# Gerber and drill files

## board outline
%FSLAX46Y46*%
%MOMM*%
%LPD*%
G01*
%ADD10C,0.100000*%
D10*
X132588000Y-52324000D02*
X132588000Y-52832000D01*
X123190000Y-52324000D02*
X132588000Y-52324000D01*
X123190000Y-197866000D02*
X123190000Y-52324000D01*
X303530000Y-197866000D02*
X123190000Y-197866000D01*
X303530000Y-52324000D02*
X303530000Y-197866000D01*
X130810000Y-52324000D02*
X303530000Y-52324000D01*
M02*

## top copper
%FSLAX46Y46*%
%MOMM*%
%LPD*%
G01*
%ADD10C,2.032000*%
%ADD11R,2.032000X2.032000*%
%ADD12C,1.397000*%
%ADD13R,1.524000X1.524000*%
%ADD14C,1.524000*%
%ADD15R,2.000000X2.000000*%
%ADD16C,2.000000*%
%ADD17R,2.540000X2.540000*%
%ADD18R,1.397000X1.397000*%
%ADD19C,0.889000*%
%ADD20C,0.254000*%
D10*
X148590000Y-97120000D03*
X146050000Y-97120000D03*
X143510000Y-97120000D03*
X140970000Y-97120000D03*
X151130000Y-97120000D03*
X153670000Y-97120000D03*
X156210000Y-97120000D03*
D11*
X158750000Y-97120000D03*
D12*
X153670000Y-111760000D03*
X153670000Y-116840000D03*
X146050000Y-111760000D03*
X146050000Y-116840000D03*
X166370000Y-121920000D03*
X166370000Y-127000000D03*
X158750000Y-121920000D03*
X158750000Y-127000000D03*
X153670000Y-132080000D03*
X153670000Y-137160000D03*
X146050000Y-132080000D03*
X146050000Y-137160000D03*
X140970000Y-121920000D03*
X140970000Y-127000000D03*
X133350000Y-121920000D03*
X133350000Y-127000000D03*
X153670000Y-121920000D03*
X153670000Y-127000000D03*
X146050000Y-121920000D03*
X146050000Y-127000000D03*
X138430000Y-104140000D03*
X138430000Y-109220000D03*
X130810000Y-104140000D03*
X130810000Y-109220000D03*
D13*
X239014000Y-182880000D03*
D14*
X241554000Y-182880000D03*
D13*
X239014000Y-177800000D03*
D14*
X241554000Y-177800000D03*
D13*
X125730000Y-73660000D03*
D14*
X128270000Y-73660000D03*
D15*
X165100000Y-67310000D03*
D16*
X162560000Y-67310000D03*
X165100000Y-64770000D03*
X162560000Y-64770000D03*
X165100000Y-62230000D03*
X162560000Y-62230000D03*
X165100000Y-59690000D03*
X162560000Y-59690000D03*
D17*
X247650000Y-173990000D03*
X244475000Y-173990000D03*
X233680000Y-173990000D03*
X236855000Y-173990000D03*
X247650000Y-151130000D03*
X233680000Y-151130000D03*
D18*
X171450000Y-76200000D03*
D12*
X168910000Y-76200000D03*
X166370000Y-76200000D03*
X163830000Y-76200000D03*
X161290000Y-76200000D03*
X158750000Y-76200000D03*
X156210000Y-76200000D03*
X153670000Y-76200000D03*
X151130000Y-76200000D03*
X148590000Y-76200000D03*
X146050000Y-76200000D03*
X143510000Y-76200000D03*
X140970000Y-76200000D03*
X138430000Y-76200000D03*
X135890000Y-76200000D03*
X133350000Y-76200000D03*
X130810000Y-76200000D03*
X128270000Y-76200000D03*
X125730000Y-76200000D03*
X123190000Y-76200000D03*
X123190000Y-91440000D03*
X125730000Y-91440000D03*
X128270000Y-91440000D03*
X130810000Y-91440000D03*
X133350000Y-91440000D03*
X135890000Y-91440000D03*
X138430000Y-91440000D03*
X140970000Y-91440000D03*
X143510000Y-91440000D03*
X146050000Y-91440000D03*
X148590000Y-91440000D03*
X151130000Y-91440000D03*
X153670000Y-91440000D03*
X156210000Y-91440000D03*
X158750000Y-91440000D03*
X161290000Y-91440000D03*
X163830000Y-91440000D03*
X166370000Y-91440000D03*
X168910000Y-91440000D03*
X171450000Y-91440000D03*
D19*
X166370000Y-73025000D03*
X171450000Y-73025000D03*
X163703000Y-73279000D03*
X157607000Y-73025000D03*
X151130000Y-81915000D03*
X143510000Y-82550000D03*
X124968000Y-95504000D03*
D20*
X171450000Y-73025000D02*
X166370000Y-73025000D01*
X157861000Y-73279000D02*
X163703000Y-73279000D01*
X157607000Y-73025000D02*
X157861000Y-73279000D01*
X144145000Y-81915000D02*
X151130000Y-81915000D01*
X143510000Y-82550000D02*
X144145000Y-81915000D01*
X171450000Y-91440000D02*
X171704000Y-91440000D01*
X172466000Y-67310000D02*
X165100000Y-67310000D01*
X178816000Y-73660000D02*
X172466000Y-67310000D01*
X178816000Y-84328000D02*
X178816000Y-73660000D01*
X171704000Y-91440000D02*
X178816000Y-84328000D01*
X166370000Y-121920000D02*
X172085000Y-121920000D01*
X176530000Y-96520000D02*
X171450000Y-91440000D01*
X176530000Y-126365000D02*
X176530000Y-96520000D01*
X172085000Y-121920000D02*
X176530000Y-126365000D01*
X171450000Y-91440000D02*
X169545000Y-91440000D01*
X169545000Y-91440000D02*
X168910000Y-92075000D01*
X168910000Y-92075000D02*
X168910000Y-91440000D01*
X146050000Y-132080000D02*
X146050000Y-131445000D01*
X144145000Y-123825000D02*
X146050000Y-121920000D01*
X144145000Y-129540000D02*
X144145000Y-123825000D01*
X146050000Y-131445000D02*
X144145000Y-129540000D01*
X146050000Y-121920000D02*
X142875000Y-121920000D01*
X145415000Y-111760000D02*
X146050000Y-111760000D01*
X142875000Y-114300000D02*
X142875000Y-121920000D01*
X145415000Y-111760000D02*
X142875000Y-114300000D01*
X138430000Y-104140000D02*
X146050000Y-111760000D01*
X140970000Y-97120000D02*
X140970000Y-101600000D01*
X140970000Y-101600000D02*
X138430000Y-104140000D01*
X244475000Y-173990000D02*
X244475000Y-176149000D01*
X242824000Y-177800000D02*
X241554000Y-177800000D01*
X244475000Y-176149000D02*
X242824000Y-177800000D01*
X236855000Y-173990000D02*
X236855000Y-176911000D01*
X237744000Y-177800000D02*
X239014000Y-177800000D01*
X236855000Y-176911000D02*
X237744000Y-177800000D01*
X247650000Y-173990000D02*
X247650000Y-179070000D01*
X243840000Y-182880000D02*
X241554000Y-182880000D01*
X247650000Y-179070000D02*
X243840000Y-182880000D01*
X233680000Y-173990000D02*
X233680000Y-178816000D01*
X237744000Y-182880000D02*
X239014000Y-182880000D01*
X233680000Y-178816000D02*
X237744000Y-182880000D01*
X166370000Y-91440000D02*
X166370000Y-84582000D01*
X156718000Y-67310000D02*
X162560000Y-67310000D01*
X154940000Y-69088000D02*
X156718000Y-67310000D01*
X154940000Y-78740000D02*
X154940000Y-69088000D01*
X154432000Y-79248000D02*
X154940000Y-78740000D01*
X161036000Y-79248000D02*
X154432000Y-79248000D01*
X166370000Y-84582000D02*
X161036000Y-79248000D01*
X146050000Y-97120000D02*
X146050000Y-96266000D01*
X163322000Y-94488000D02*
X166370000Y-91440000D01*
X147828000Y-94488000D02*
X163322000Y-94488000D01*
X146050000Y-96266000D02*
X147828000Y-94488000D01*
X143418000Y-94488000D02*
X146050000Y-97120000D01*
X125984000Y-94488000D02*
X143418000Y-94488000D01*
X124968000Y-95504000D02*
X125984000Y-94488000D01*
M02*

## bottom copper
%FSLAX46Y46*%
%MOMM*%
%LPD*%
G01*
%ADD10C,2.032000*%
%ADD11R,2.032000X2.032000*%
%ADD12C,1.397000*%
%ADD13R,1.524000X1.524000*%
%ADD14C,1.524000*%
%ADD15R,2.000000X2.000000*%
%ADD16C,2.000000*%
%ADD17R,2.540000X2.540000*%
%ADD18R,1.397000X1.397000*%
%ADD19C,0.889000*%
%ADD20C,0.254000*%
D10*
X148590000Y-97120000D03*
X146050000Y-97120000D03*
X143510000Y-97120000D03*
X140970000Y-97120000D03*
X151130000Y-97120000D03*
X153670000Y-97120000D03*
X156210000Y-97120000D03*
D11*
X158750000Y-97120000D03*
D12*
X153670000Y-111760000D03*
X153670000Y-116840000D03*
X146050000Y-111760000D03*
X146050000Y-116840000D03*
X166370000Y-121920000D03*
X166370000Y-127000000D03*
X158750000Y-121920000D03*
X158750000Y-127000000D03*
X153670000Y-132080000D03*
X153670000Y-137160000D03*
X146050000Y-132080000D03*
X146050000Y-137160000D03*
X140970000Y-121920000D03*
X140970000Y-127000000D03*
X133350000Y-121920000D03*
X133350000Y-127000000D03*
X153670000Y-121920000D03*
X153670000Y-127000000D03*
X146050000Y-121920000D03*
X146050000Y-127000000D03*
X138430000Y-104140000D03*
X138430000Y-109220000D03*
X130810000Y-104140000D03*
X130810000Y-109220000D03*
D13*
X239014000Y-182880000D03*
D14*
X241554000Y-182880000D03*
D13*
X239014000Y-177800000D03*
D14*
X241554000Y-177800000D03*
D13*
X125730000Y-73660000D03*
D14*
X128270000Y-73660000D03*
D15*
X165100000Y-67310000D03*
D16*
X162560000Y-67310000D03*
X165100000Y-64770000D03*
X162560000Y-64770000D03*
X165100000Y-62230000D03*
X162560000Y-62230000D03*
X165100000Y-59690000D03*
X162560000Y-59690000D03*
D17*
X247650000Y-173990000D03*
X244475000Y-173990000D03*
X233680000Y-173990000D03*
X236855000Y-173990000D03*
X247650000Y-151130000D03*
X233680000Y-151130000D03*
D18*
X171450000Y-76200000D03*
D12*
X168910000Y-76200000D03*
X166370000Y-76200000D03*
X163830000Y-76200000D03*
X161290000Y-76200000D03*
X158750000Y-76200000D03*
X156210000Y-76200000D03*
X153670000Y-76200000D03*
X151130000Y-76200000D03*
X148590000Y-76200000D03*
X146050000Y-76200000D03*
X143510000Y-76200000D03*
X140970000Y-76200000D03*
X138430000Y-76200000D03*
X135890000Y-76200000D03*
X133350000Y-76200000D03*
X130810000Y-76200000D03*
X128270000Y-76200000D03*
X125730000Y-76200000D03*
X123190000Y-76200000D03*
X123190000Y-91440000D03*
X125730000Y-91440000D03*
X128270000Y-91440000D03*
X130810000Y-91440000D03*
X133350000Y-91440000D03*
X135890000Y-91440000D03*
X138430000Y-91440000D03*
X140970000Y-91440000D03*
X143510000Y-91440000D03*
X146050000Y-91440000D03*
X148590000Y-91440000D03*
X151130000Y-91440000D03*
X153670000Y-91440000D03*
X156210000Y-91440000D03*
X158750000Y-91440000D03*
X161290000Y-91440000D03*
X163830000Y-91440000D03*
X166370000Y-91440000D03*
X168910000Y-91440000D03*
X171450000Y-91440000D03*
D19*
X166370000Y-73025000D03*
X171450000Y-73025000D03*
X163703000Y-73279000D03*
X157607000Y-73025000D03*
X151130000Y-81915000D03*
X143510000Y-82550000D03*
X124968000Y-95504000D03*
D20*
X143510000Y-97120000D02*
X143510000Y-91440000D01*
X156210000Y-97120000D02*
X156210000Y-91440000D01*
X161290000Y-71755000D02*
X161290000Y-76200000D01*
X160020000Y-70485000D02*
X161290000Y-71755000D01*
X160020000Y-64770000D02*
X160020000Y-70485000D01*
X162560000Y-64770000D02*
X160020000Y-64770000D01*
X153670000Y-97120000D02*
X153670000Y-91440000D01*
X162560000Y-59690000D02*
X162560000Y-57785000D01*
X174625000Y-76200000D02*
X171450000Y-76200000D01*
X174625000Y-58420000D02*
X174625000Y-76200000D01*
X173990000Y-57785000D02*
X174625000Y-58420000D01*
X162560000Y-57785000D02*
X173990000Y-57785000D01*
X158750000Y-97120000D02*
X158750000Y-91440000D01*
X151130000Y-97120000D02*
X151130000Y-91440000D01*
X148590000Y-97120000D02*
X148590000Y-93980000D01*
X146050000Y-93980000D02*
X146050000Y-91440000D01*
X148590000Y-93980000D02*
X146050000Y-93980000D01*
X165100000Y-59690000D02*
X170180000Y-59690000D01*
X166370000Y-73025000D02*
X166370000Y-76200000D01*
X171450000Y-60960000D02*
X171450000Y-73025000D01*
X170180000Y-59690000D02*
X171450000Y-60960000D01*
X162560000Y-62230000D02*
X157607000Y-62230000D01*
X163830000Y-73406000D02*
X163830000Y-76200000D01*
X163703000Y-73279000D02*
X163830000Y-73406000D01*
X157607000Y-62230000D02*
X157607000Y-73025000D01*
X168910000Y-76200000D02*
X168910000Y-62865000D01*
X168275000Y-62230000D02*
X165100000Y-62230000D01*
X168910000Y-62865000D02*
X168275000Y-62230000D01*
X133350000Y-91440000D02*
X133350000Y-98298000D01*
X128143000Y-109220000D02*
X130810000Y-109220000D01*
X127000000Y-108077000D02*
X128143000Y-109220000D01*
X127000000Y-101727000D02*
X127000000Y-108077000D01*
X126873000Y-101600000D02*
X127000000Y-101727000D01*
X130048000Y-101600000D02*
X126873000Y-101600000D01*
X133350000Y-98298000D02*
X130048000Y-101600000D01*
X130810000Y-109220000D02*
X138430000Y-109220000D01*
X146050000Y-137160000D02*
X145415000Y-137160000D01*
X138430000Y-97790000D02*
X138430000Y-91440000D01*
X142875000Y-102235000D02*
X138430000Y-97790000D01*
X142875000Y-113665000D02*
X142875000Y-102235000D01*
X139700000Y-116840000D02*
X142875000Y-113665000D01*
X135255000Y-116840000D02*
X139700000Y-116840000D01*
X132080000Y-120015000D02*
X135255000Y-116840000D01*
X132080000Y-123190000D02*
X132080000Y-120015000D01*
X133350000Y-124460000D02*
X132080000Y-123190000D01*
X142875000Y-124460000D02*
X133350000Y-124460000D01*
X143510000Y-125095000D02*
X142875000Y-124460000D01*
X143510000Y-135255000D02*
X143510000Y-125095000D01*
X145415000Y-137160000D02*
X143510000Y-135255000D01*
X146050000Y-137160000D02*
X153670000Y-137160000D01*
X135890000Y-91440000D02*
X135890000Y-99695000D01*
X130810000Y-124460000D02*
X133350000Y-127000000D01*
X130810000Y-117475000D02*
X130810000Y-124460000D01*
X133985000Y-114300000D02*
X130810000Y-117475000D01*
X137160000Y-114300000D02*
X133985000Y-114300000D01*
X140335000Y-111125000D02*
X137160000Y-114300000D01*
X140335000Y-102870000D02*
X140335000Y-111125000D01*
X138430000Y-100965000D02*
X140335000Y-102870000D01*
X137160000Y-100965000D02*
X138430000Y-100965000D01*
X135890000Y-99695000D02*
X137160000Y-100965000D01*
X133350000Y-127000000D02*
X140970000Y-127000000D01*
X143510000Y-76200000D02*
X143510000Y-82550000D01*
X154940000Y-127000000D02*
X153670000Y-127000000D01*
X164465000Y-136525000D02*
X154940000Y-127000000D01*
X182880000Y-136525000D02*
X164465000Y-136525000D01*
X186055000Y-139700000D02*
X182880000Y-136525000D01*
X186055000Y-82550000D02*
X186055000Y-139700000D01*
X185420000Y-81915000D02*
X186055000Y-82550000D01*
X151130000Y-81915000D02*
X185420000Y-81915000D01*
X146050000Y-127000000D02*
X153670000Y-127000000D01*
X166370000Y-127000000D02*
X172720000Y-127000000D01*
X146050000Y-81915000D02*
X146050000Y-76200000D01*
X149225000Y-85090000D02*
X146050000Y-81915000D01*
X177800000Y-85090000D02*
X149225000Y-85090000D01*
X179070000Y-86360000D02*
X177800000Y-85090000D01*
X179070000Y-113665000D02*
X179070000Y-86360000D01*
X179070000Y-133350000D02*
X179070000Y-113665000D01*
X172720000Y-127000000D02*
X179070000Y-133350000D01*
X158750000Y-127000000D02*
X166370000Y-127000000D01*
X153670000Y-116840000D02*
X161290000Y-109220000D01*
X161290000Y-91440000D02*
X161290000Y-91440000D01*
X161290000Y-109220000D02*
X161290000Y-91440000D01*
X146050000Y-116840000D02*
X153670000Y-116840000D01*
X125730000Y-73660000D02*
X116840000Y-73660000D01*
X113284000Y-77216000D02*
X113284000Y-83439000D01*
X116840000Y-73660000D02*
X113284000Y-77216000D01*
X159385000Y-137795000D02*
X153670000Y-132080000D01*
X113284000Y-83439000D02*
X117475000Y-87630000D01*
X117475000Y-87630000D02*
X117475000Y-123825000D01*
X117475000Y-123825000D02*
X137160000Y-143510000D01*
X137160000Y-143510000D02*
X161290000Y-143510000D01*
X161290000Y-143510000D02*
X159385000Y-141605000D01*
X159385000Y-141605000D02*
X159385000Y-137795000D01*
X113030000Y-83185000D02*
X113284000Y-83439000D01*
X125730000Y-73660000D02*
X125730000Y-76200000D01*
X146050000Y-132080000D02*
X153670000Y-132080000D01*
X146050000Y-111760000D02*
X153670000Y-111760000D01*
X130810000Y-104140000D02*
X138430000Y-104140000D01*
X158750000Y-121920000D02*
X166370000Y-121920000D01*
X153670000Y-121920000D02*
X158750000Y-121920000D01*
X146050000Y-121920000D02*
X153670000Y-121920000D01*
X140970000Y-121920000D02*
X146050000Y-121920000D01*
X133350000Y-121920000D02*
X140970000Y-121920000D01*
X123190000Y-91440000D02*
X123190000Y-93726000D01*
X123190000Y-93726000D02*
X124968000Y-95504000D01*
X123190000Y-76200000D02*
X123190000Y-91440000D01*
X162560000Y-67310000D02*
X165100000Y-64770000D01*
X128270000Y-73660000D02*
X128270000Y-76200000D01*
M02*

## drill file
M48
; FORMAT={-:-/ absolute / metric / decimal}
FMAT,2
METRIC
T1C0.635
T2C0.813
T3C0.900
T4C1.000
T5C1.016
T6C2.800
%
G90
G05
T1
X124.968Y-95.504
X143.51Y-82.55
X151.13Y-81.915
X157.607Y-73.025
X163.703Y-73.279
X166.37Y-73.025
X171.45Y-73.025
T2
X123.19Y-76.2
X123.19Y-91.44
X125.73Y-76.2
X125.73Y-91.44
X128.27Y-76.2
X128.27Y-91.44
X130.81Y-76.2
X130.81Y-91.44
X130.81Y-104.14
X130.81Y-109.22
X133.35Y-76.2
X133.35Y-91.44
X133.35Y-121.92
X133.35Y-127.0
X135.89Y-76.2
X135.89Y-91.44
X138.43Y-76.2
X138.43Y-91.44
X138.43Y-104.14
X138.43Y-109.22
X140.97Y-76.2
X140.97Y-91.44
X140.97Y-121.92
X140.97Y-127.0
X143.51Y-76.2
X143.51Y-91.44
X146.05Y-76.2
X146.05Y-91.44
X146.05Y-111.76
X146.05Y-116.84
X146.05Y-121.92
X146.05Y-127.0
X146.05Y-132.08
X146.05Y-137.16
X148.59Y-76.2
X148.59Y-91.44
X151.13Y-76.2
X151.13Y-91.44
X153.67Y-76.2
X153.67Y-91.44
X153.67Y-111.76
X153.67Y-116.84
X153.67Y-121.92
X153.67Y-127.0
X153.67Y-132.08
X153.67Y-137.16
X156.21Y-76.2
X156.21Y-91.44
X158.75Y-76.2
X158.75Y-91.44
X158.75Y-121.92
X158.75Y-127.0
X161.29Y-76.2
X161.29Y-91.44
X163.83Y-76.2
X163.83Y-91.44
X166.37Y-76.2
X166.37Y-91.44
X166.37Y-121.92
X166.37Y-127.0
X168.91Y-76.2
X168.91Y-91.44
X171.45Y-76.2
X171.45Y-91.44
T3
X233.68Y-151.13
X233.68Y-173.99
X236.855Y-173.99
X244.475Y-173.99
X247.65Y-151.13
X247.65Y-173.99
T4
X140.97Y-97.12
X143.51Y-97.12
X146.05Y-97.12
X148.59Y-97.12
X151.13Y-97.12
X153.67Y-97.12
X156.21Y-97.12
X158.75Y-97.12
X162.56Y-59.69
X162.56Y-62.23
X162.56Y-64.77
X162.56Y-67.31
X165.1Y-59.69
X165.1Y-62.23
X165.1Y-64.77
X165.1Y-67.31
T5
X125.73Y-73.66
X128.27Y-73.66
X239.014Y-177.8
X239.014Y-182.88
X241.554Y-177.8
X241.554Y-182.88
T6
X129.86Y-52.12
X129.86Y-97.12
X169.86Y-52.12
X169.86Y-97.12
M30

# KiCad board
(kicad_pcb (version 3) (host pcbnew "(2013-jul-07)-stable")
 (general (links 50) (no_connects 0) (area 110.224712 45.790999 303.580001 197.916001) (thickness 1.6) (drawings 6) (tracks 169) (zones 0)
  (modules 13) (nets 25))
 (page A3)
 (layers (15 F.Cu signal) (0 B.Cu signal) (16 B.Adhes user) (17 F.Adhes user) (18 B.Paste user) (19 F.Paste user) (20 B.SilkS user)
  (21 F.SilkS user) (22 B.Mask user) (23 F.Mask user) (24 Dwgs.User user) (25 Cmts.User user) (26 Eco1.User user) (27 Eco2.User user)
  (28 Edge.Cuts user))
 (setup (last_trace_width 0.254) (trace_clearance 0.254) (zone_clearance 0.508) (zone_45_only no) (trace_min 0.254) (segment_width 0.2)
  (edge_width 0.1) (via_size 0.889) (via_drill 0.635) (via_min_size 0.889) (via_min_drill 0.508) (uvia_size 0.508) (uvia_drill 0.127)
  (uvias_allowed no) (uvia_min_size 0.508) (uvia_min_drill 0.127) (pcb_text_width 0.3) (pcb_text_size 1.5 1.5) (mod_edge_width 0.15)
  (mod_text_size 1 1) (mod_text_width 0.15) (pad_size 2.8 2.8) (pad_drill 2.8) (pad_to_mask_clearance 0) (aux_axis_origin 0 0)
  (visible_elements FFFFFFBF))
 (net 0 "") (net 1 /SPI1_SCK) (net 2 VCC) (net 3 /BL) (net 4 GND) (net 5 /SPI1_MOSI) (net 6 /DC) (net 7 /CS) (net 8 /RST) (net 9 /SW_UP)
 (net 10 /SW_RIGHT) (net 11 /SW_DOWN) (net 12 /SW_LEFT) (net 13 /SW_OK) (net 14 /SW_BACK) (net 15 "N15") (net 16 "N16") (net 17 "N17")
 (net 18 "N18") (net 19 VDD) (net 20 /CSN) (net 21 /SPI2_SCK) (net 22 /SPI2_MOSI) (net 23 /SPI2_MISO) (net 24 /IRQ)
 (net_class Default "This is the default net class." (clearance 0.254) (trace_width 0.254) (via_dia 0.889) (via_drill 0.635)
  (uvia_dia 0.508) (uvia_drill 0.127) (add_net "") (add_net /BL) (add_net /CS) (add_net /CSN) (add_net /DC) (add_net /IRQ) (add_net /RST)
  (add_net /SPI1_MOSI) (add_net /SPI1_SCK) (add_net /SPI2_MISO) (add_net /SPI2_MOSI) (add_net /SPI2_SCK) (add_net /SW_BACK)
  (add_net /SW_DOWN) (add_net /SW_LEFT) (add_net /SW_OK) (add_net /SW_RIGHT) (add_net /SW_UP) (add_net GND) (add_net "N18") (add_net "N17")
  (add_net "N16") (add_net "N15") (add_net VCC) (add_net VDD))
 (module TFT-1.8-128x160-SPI (layer F.Cu) (at 149.86 71.12 270)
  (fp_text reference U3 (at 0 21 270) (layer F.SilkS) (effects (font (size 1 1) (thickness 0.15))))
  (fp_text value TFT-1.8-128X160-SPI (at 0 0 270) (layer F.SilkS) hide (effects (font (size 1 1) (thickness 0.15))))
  (pad 5 thru_hole circle (at 26 1.27 270) (size 2.032 2.032) (drill 1) (layers *.Cu *.Mask F.SilkS) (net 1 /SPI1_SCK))
  (pad 6 thru_hole circle (at 26 3.81 270) (size 2.032 2.032) (drill 1) (layers *.Cu *.Mask F.SilkS) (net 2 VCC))
  (pad 7 thru_hole circle (at 26 6.35 270) (size 2.032 2.032) (drill 1) (layers *.Cu *.Mask F.SilkS) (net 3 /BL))
  (pad 8 thru_hole circle (at 26 8.89 270) (size 2.032 2.032) (drill 1) (layers *.Cu *.Mask F.SilkS) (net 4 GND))
  (pad 4 thru_hole circle (at 26 -1.27 270) (size 2.032 2.032) (drill 1) (layers *.Cu *.Mask F.SilkS) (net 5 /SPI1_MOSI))
  (pad 3 thru_hole circle (at 26 -3.81 270) (size 2.032 2.032) (drill 1) (layers *.Cu *.Mask F.SilkS) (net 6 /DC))
  (pad 2 thru_hole circle (at 26 -6.35 270) (size 2.032 2.032) (drill 1) (layers *.Cu *.Mask F.SilkS) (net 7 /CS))
  (pad 1 thru_hole rect (at 26 -8.89 270) (size 2.032 2.032) (drill 1) (layers *.Cu *.Mask F.SilkS) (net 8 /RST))
  (pad "" np_thru_hole circle (at -19 20 270) (size 2.8 2.8) (drill 2.8) (layers *.Cu *.Mask F.SilkS))
  (pad "" np_thru_hole circle (at 26 20 270) (size 2.8 2.8) (drill 2.8) (layers *.Cu *.Mask F.SilkS))
  (pad "" np_thru_hole circle (at 26 -20 270) (size 2.8 2.8) (drill 2.8) (layers *.Cu *.Mask F.SilkS))
  (pad "" np_thru_hole circle (at -19 -20 270) (size 2.8 2.8) (drill 2.8) (layers *.Cu *.Mask F.SilkS)))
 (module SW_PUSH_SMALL (layer F.Cu) (at 149.86 114.3)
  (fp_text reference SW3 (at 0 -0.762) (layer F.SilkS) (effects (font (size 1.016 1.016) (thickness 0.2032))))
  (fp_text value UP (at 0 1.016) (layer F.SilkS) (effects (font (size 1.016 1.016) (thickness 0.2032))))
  (pad 1 thru_hole circle (at 3.81 -2.54) (size 1.397 1.397) (drill 0.8128) (layers *.Cu *.Mask F.SilkS) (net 4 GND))
  (pad 2 thru_hole circle (at 3.81 2.54) (size 1.397 1.397) (drill 0.8128) (layers *.Cu *.Mask F.SilkS) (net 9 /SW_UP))
  (pad 1 thru_hole circle (at -3.81 -2.54) (size 1.397 1.397) (drill 0.8128) (layers *.Cu *.Mask F.SilkS) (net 4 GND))
  (pad 2 thru_hole circle (at -3.81 2.54) (size 1.397 1.397) (drill 0.8128) (layers *.Cu *.Mask F.SilkS) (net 9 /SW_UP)))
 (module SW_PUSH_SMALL (layer F.Cu) (at 162.56 124.46)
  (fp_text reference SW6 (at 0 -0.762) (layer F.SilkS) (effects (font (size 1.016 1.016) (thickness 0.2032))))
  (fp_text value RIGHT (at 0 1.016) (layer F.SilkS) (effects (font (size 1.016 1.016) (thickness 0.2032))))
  (pad 1 thru_hole circle (at 3.81 -2.54) (size 1.397 1.397) (drill 0.8128) (layers *.Cu *.Mask F.SilkS) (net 4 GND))
  (pad 2 thru_hole circle (at 3.81 2.54) (size 1.397 1.397) (drill 0.8128) (layers *.Cu *.Mask F.SilkS) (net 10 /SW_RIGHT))
  (pad 1 thru_hole circle (at -3.81 -2.54) (size 1.397 1.397) (drill 0.8128) (layers *.Cu *.Mask F.SilkS) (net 4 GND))
  (pad 2 thru_hole circle (at -3.81 2.54) (size 1.397 1.397) (drill 0.8128) (layers *.Cu *.Mask F.SilkS) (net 10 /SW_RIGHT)))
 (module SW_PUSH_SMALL (layer F.Cu) (at 149.86 134.62)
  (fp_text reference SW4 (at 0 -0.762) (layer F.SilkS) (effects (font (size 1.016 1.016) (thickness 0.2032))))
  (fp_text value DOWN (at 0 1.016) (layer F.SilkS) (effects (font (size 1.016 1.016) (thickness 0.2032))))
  (pad 1 thru_hole circle (at 3.81 -2.54) (size 1.397 1.397) (drill 0.8128) (layers *.Cu *.Mask F.SilkS) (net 4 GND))
  (pad 2 thru_hole circle (at 3.81 2.54) (size 1.397 1.397) (drill 0.8128) (layers *.Cu *.Mask F.SilkS) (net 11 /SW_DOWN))
  (pad 1 thru_hole circle (at -3.81 -2.54) (size 1.397 1.397) (drill 0.8128) (layers *.Cu *.Mask F.SilkS) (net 4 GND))
  (pad 2 thru_hole circle (at -3.81 2.54) (size 1.397 1.397) (drill 0.8128) (layers *.Cu *.Mask F.SilkS) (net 11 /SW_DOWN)))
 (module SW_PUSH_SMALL (layer F.Cu) (at 137.16 124.46)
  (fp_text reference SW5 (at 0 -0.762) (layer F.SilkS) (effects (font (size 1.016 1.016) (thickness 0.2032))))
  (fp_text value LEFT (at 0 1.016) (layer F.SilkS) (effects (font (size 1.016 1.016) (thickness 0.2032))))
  (pad 1 thru_hole circle (at 3.81 -2.54) (size 1.397 1.397) (drill 0.8128) (layers *.Cu *.Mask F.SilkS) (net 4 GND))
  (pad 2 thru_hole circle (at 3.81 2.54) (size 1.397 1.397) (drill 0.8128) (layers *.Cu *.Mask F.SilkS) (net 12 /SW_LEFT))
  (pad 1 thru_hole circle (at -3.81 -2.54) (size 1.397 1.397) (drill 0.8128) (layers *.Cu *.Mask F.SilkS) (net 4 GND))
  (pad 2 thru_hole circle (at -3.81 2.54) (size 1.397 1.397) (drill 0.8128) (layers *.Cu *.Mask F.SilkS) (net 12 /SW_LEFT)))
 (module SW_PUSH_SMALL (layer F.Cu) (at 149.86 124.46)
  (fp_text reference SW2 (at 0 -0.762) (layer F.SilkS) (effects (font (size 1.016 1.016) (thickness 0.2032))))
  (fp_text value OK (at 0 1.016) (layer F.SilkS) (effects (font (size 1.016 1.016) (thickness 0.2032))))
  (pad 1 thru_hole circle (at 3.81 -2.54) (size 1.397 1.397) (drill 0.8128) (layers *.Cu *.Mask F.SilkS) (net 4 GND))
  (pad 2 thru_hole circle (at 3.81 2.54) (size 1.397 1.397) (drill 0.8128) (layers *.Cu *.Mask F.SilkS) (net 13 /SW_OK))
  (pad 1 thru_hole circle (at -3.81 -2.54) (size 1.397 1.397) (drill 0.8128) (layers *.Cu *.Mask F.SilkS) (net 4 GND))
  (pad 2 thru_hole circle (at -3.81 2.54) (size 1.397 1.397) (drill 0.8128) (layers *.Cu *.Mask F.SilkS) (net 13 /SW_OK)))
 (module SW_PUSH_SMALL (layer F.Cu) (at 134.62 106.68)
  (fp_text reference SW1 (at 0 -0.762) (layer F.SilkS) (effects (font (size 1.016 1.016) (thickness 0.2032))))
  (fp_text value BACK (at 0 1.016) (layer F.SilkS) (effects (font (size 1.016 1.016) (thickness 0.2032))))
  (pad 1 thru_hole circle (at 3.81 -2.54) (size 1.397 1.397) (drill 0.8128) (layers *.Cu *.Mask F.SilkS) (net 4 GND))
  (pad 2 thru_hole circle (at 3.81 2.54) (size 1.397 1.397) (drill 0.8128) (layers *.Cu *.Mask F.SilkS) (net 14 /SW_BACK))
  (pad 1 thru_hole circle (at -3.81 -2.54) (size 1.397 1.397) (drill 0.8128) (layers *.Cu *.Mask F.SilkS) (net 4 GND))
  (pad 2 thru_hole circle (at -3.81 2.54) (size 1.397 1.397) (drill 0.8128) (layers *.Cu *.Mask F.SilkS) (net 14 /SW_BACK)))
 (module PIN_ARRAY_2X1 (layer F.Cu) (at 240.284 182.88)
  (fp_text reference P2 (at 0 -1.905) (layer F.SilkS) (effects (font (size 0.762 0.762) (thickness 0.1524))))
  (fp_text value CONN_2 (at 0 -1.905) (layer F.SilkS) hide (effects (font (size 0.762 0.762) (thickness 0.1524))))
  (pad 1 thru_hole rect (at -1.27 0) (size 1.524 1.524) (drill 1.016) (layers *.Cu *.Mask F.SilkS) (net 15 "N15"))
  (pad 2 thru_hole circle (at 1.27 0) (size 1.524 1.524) (drill 1.016) (layers *.Cu *.Mask F.SilkS) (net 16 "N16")))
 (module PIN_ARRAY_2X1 (layer F.Cu) (at 240.284 177.8)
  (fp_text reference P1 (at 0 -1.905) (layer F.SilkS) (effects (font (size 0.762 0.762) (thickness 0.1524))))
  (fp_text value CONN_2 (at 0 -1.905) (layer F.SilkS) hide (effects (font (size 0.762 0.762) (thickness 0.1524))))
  (pad 1 thru_hole rect (at -1.27 0) (size 1.524 1.524) (drill 1.016) (layers *.Cu *.Mask F.SilkS) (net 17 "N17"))
  (pad 2 thru_hole circle (at 1.27 0) (size 1.524 1.524) (drill 1.016) (layers *.Cu *.Mask F.SilkS) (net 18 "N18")))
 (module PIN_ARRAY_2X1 (layer F.Cu) (at 127 73.66)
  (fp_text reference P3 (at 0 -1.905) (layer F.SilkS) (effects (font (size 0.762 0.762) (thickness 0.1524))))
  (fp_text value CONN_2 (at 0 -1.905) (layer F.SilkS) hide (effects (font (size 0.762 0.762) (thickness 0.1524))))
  (pad 1 thru_hole rect (at -1.27 0) (size 1.524 1.524) (drill 1.016) (layers *.Cu *.Mask F.SilkS) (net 4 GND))
  (pad 2 thru_hole circle (at 1.27 0) (size 1.524 1.524) (drill 1.016) (layers *.Cu *.Mask F.SilkS) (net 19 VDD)))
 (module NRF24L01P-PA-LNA (layer F.Cu) (at 165.1 63.5 90)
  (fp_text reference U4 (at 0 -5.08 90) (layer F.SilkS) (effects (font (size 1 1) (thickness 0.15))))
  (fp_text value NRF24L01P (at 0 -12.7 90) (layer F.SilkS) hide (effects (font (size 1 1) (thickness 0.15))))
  (pad 1 thru_hole rect (at -3.81 0 90) (size 2 2) (drill 1) (layers *.Cu *.Mask F.SilkS) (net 4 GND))
  (pad 2 thru_hole circle (at -3.81 -2.54 90) (size 2 2) (drill 1) (layers *.Cu *.Mask F.SilkS) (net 2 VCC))
  (pad 3 thru_hole circle (at -1.27 0 90) (size 2 2) (drill 1) (layers *.Cu *.Mask F.SilkS) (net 2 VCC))
  (pad 4 thru_hole circle (at -1.27 -2.54 90) (size 2 2) (drill 1) (layers *.Cu *.Mask F.SilkS) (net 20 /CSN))
  (pad 5 thru_hole circle (at 1.27 0 90) (size 2 2) (drill 1) (layers *.Cu *.Mask F.SilkS) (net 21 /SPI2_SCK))
  (pad 6 thru_hole circle (at 1.27 -2.54 90) (size 2 2) (drill 1) (layers *.Cu *.Mask F.SilkS) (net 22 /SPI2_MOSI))
  (pad 7 thru_hole circle (at 3.81 0 90) (size 2 2) (drill 1) (layers *.Cu *.Mask F.SilkS) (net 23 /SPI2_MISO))
  (pad 8 thru_hole circle (at 3.81 -2.54 90) (size 2 2) (drill 1) (layers *.Cu *.Mask F.SilkS) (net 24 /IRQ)))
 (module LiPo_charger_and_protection (layer F.Cu) (at 240.665 162.56 270)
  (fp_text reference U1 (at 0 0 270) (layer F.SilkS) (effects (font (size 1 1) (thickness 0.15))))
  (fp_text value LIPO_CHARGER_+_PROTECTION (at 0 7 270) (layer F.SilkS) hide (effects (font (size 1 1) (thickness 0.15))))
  (pad 3 thru_hole rect (at 11.43 -6.985 270) (size 2.54 2.54) (drill 0.9) (layers *.Cu *.Mask F.SilkS) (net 16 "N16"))
  (pad 1 thru_hole rect (at 11.43 -3.81 270) (size 2.54 2.54) (drill 0.9) (layers *.Cu *.Mask F.SilkS) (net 18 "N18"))
  (pad 4 thru_hole rect (at 11.43 6.985 270) (size 2.54 2.54) (drill 0.9) (layers *.Cu *.Mask F.SilkS) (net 15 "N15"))
  (pad 2 thru_hole rect (at 11.43 3.81 270) (size 2.54 2.54) (drill 0.9) (layers *.Cu *.Mask F.SilkS) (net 17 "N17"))
  (pad 5 thru_hole rect (at -11.43 -6.985 270) (size 2.54 2.54) (drill 0.9) (layers *.Cu *.Mask F.SilkS))
  (pad 6 thru_hole rect (at -11.43 6.985 270) (size 2.54 2.54) (drill 0.9) (layers *.Cu *.Mask F.SilkS)))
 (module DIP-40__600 (layer F.Cu) (at 147.32 83.82 180)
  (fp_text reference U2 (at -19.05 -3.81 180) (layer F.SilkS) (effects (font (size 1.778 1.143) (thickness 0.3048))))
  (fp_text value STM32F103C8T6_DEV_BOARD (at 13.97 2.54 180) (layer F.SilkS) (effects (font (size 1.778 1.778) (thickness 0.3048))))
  (pad 1 thru_hole rect (at -24.13 7.62 180) (size 1.397 1.397) (drill 0.8128) (layers *.Cu *.Mask F.SilkS) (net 24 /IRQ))
  (pad 2 thru_hole circle (at -21.59 7.62 180) (size 1.397 1.397) (drill 0.8128) (layers *.Cu *.Mask F.SilkS) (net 21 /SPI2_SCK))
  (pad 3 thru_hole circle (at -19.05 7.62 180) (size 1.397 1.397) (drill 0.8128) (layers *.Cu *.Mask F.SilkS) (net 23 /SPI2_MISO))
  (pad 4 thru_hole circle (at -16.51 7.62 180) (size 1.397 1.397) (drill 0.8128) (layers *.Cu *.Mask F.SilkS) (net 22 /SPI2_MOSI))
  (pad 5 thru_hole circle (at -13.97 7.62 180) (size 1.397 1.397) (drill 0.8128) (layers *.Cu *.Mask F.SilkS) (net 20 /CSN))
  (pad 6 thru_hole circle (at -11.43 7.62 180) (size 1.397 1.397) (drill 0.8128) (layers *.Cu *.Mask F.SilkS))
  (pad 7 thru_hole circle (at -8.89 7.62 180) (size 1.397 1.397) (drill 0.8128) (layers *.Cu *.Mask F.SilkS))
  (pad 8 thru_hole circle (at -6.35 7.62 180) (size 1.397 1.397) (drill 0.8128) (layers *.Cu *.Mask F.SilkS))
  (pad 9 thru_hole circle (at -3.81 7.62 180) (size 1.397 1.397) (drill 0.8128) (layers *.Cu *.Mask F.SilkS))
  (pad 10 thru_hole circle (at -1.27 7.62 180) (size 1.397 1.397) (drill 0.8128) (layers *.Cu *.Mask F.SilkS))
  (pad 11 thru_hole circle (at 1.27 7.62 180) (size 1.397 1.397) (drill 0.8128) (layers *.Cu *.Mask F.SilkS) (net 10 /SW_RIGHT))
  (pad 12 thru_hole circle (at 3.81 7.62 180) (size 1.397 1.397) (drill 0.8128) (layers *.Cu *.Mask F.SilkS) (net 13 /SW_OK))
  (pad 13 thru_hole circle (at 6.35 7.62 180) (size 1.397 1.397) (drill 0.8128) (layers *.Cu *.Mask F.SilkS))
  (pad 14 thru_hole circle (at 8.89 7.62 180) (size 1.397 1.397) (drill 0.8128) (layers *.Cu *.Mask F.SilkS))
  (pad 15 thru_hole circle (at 11.43 7.62 180) (size 1.397 1.397) (drill 0.8128) (layers *.Cu *.Mask F.SilkS))
  (pad 16 thru_hole circle (at 13.97 7.62 180) (size 1.397 1.397) (drill 0.8128) (layers *.Cu *.Mask F.SilkS))
  (pad 17 thru_hole circle (at 16.51 7.62 180) (size 1.397 1.397) (drill 0.8128) (layers *.Cu *.Mask F.SilkS))
  (pad 18 thru_hole circle (at 19.05 7.62 180) (size 1.397 1.397) (drill 0.8128) (layers *.Cu *.Mask F.SilkS) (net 19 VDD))
  (pad 19 thru_hole circle (at 21.59 7.62 180) (size 1.397 1.397) (drill 0.8128) (layers *.Cu *.Mask F.SilkS) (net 4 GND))
  (pad 20 thru_hole circle (at 24.13 7.62 180) (size 1.397 1.397) (drill 0.8128) (layers *.Cu *.Mask F.SilkS) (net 2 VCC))
  (pad 21 thru_hole circle (at 24.13 -7.62 180) (size 1.397 1.397) (drill 0.8128) (layers *.Cu *.Mask F.SilkS) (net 2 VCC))
  (pad 22 thru_hole circle (at 21.59 -7.62 180) (size 1.397 1.397) (drill 0.8128) (layers *.Cu *.Mask F.SilkS))
  (pad 23 thru_hole circle (at 19.05 -7.62 180) (size 1.397 1.397) (drill 0.8128) (layers *.Cu *.Mask F.SilkS))
  (pad 24 thru_hole circle (at 16.51 -7.62 180) (size 1.397 1.397) (drill 0.8128) (layers *.Cu *.Mask F.SilkS))
  (pad 25 thru_hole circle (at 13.97 -7.62 180) (size 1.397 1.397) (drill 0.8128) (layers *.Cu *.Mask F.SilkS) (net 14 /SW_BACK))
  (pad 26 thru_hole circle (at 11.43 -7.62 180) (size 1.397 1.397) (drill 0.8128) (layers *.Cu *.Mask F.SilkS) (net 12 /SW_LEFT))
  (pad 27 thru_hole circle (at 8.89 -7.62 180) (size 1.397 1.397) (drill 0.8128) (layers *.Cu *.Mask F.SilkS) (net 11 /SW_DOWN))
  (pad 28 thru_hole circle (at 6.35 -7.62 180) (size 1.397 1.397) (drill 0.8128) (layers *.Cu *.Mask F.SilkS))
  (pad 29 thru_hole circle (at 3.81 -7.62 180) (size 1.397 1.397) (drill 0.8128) (layers *.Cu *.Mask F.SilkS) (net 3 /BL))
  (pad 30 thru_hole circle (at 1.27 -7.62 180) (size 1.397 1.397) (drill 0.8128) (layers *.Cu *.Mask F.SilkS) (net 1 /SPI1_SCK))
  (pad 31 thru_hole circle (at -1.27 -7.62 180) (size 1.397 1.397) (drill 0.8128) (layers *.Cu *.Mask F.SilkS))
  (pad 32 thru_hole circle (at -3.81 -7.62 180) (size 1.397 1.397) (drill 0.8128) (layers *.Cu *.Mask F.SilkS) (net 5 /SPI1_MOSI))
  (pad 33 thru_hole circle (at -6.35 -7.62 180) (size 1.397 1.397) (drill 0.8128) (layers *.Cu *.Mask F.SilkS) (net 6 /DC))
  (pad 34 thru_hole circle (at -8.89 -7.62 180) (size 1.397 1.397) (drill 0.8128) (layers *.Cu *.Mask F.SilkS) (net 7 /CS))
  (pad 35 thru_hole circle (at -11.43 -7.62 180) (size 1.397 1.397) (drill 0.8128) (layers *.Cu *.Mask F.SilkS) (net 8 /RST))
  (pad 36 thru_hole circle (at -13.97 -7.62 180) (size 1.397 1.397) (drill 0.8128) (layers *.Cu *.Mask F.SilkS) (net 9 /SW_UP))
  (pad 37 thru_hole circle (at -16.51 -7.62 180) (size 1.397 1.397) (drill 0.8128) (layers *.Cu *.Mask F.SilkS))
  (pad 38 thru_hole circle (at -19.05 -7.62 180) (size 1.397 1.397) (drill 0.8128) (layers *.Cu *.Mask F.SilkS) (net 2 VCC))
  (pad 39 thru_hole circle (at -21.59 -7.62 180) (size 1.397 1.397) (drill 0.8128) (layers *.Cu *.Mask F.SilkS) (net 4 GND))
  (pad 40 thru_hole circle (at -24.13 -7.62 180) (size 1.397 1.397) (drill 0.8128) (layers *.Cu *.Mask F.SilkS) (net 4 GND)))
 (gr_line (start 132.588 52.324) (end 132.588 52.832) (angle 90) (layer Edge.Cuts) (width 0.1))
 (gr_line (start 123.19 52.324) (end 132.588 52.324) (angle 90) (layer Edge.Cuts) (width 0.1))
 (gr_line (start 123.19 197.866) (end 123.19 52.324) (angle 90) (layer Edge.Cuts) (width 0.1))
 (gr_line (start 303.53 197.866) (end 123.19 197.866) (angle 90) (layer Edge.Cuts) (width 0.1))
 (gr_line (start 303.53 52.324) (end 303.53 197.866) (angle 90) (layer Edge.Cuts) (width 0.1))
 (gr_line (start 130.81 52.324) (end 303.53 52.324) (angle 90) (layer Edge.Cuts) (width 0.1))
 (segment (start 143.51 97.12) (end 143.51 91.44) (width 0.254) (layer B.Cu) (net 3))
 (segment (start 156.21 97.12) (end 156.21 91.44) (width 0.254) (layer B.Cu) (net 7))
 (segment (start 161.29 71.755) (end 161.29 76.2) (width 0.254) (layer B.Cu) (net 20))
 (segment (start 160.02 70.485) (end 161.29 71.755) (width 0.254) (layer B.Cu) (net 20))
 (segment (start 160.02 64.77) (end 160.02 70.485) (width 0.254) (layer B.Cu) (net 20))
 (segment (start 162.56 64.77) (end 160.02 64.77) (width 0.254) (layer B.Cu) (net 20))
 (segment (start 153.67 97.12) (end 153.67 91.44) (width 0.254) (layer B.Cu) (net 6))
 (segment (start 162.56 59.69) (end 162.56 57.785) (width 0.254) (layer B.Cu) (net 24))
 (segment (start 174.625 76.2) (end 171.45 76.2) (width 0.254) (layer B.Cu) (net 24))
 (segment (start 174.625 58.42) (end 174.625 76.2) (width 0.254) (layer B.Cu) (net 24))
 (segment (start 173.99 57.785) (end 174.625 58.42) (width 0.254) (layer B.Cu) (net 24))
 (segment (start 162.56 57.785) (end 173.99 57.785) (width 0.254) (layer B.Cu) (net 24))
 (segment (start 158.75 97.12) (end 158.75 91.44) (width 0.254) (layer B.Cu) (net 8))
 (segment (start 151.13 97.12) (end 151.13 91.44) (width 0.254) (layer B.Cu) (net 5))
 (segment (start 148.59 97.12) (end 148.59 93.98) (width 0.254) (layer B.Cu) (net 1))
 (segment (start 146.05 93.98) (end 146.05 91.44) (width 0.254) (layer B.Cu) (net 1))
 (segment (start 148.59 93.98) (end 146.05 93.98) (width 0.254) (layer B.Cu) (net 1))
 (segment (start 165.1 59.69) (end 170.18 59.69) (width 0.254) (layer B.Cu) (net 23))
 (segment (start 166.37 73.025) (end 166.37 76.2) (width 0.254) (layer B.Cu) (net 23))
 (via (at 166.37 73.025) (size 0.889) (layers F.Cu B.Cu) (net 23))
 (segment (start 171.45 73.025) (end 166.37 73.025) (width 0.254) (layer F.Cu) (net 23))
 (via (at 171.45 73.025) (size 0.889) (layers F.Cu B.Cu) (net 23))
 (segment (start 171.45 60.96) (end 171.45 73.025) (width 0.254) (layer B.Cu) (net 23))
 (segment (start 170.18 59.69) (end 171.45 60.96) (width 0.254) (layer B.Cu) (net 23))
 (segment (start 162.56 62.23) (end 157.607 62.23) (width 0.254) (layer B.Cu) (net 22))
 (segment (start 163.83 73.406) (end 163.83 76.2) (width 0.254) (layer B.Cu) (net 22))
 (segment (start 163.703 73.279) (end 163.83 73.406) (width 0.254) (layer B.Cu) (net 22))
 (via (at 163.703 73.279) (size 0.889) (layers F.Cu B.Cu) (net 22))
 (segment (start 157.861 73.279) (end 163.703 73.279) (width 0.254) (layer F.Cu) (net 22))
 (segment (start 157.607 73.025) (end 157.861 73.279) (width 0.254) (layer F.Cu) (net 22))
 (via (at 157.607 73.025) (size 0.889) (layers F.Cu B.Cu) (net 22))
 (segment (start 157.607 62.23) (end 157.607 73.025) (width 0.254) (layer B.Cu) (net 22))
 (segment (start 168.91 76.2) (end 168.91 62.865) (width 0.254) (layer B.Cu) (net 21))
 (segment (start 168.275 62.23) (end 165.1 62.23) (width 0.254) (layer B.Cu) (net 21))
 (segment (start 168.91 62.865) (end 168.275 62.23) (width 0.254) (layer B.Cu) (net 21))
 (segment (start 133.35 91.44) (end 133.35 98.298) (width 0.254) (layer B.Cu) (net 14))
 (segment (start 128.143 109.22) (end 130.81 109.22) (width 0.254) (layer B.Cu) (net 14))
 (segment (start 127 108.077) (end 128.143 109.22) (width 0.254) (layer B.Cu) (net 14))
 (segment (start 127 101.727) (end 127 108.077) (width 0.254) (layer B.Cu) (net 14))
 (segment (start 126.873 101.6) (end 127 101.727) (width 0.254) (layer B.Cu) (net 14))
 (segment (start 130.048 101.6) (end 126.873 101.6) (width 0.254) (layer B.Cu) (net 14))
 (segment (start 133.35 98.298) (end 130.048 101.6) (width 0.254) (layer B.Cu) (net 14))
 (segment (start 130.81 109.22) (end 138.43 109.22) (width 0.254) (layer B.Cu) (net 14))
 (segment (start 146.05 137.16) (end 145.415 137.16) (width 0.254) (layer B.Cu) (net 11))
 (segment (start 138.43 97.79) (end 138.43 91.44) (width 0.254) (layer B.Cu) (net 11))
 (segment (start 142.875 102.235) (end 138.43 97.79) (width 0.254) (layer B.Cu) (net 11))
 (segment (start 142.875 113.665) (end 142.875 102.235) (width 0.254) (layer B.Cu) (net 11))
 (segment (start 139.7 116.84) (end 142.875 113.665) (width 0.254) (layer B.Cu) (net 11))
 (segment (start 135.255 116.84) (end 139.7 116.84) (width 0.254) (layer B.Cu) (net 11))
 (segment (start 132.08 120.015) (end 135.255 116.84) (width 0.254) (layer B.Cu) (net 11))
 (segment (start 132.08 123.19) (end 132.08 120.015) (width 0.254) (layer B.Cu) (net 11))
 (segment (start 133.35 124.46) (end 132.08 123.19) (width 0.254) (layer B.Cu) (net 11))
 (segment (start 142.875 124.46) (end 133.35 124.46) (width 0.254) (layer B.Cu) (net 11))
 (segment (start 143.51 125.095) (end 142.875 124.46) (width 0.254) (layer B.Cu) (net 11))
 (segment (start 143.51 135.255) (end 143.51 125.095) (width 0.254) (layer B.Cu) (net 11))
 (segment (start 145.415 137.16) (end 143.51 135.255) (width 0.254) (layer B.Cu) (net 11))
 (segment (start 146.05 137.16) (end 153.67 137.16) (width 0.254) (layer B.Cu) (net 11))
 (segment (start 135.89 91.44) (end 135.89 99.695) (width 0.254) (layer B.Cu) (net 12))
 (segment (start 130.81 124.46) (end 133.35 127) (width 0.254) (layer B.Cu) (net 12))
 (segment (start 130.81 117.475) (end 130.81 124.46) (width 0.254) (layer B.Cu) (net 12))
 (segment (start 133.985 114.3) (end 130.81 117.475) (width 0.254) (layer B.Cu) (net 12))
 (segment (start 137.16 114.3) (end 133.985 114.3) (width 0.254) (layer B.Cu) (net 12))
 (segment (start 140.335 111.125) (end 137.16 114.3) (width 0.254) (layer B.Cu) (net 12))
 (segment (start 140.335 102.87) (end 140.335 111.125) (width 0.254) (layer B.Cu) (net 12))
 (segment (start 138.43 100.965) (end 140.335 102.87) (width 0.254) (layer B.Cu) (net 12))
 (segment (start 137.16 100.965) (end 138.43 100.965) (width 0.254) (layer B.Cu) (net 12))
 (segment (start 135.89 99.695) (end 137.16 100.965) (width 0.254) (layer B.Cu) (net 12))
 (segment (start 133.35 127) (end 140.97 127) (width 0.254) (layer B.Cu) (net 12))
 (segment (start 143.51 76.2) (end 143.51 82.55) (width 0.254) (layer B.Cu) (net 13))
 (segment (start 154.94 127) (end 153.67 127) (width 0.254) (layer B.Cu) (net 13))
 (segment (start 164.465 136.525) (end 154.94 127) (width 0.254) (layer B.Cu) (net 13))
 (segment (start 182.88 136.525) (end 164.465 136.525) (width 0.254) (layer B.Cu) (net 13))
 (segment (start 186.055 139.7) (end 182.88 136.525) (width 0.254) (layer B.Cu) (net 13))
 (segment (start 186.055 82.55) (end 186.055 139.7) (width 0.254) (layer B.Cu) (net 13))
 (segment (start 185.42 81.915) (end 186.055 82.55) (width 0.254) (layer B.Cu) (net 13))
 (segment (start 151.13 81.915) (end 185.42 81.915) (width 0.254) (layer B.Cu) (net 13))
 (via (at 151.13 81.915) (size 0.889) (layers F.Cu B.Cu) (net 13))
 (segment (start 144.145 81.915) (end 151.13 81.915) (width 0.254) (layer F.Cu) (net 13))
 (segment (start 143.51 82.55) (end 144.145 81.915) (width 0.254) (layer F.Cu) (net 13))
 (via (at 143.51 82.55) (size 0.889) (layers F.Cu B.Cu) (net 13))
 (segment (start 146.05 127) (end 153.67 127) (width 0.254) (layer B.Cu) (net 13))
 (segment (start 166.37 127) (end 172.72 127) (width 0.254) (layer B.Cu) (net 10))
 (segment (start 146.05 81.915) (end 146.05 76.2) (width 0.254) (layer B.Cu) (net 10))
 (segment (start 149.225 85.09) (end 146.05 81.915) (width 0.254) (layer B.Cu) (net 10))
 (segment (start 177.8 85.09) (end 149.225 85.09) (width 0.254) (layer B.Cu) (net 10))
 (segment (start 179.07 86.36) (end 177.8 85.09) (width 0.254) (layer B.Cu) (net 10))
 (segment (start 179.07 113.665) (end 179.07 86.36) (width 0.254) (layer B.Cu) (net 10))
 (segment (start 179.07 133.35) (end 179.07 113.665) (width 0.254) (layer B.Cu) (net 10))
 (segment (start 172.72 127) (end 179.07 133.35) (width 0.254) (layer B.Cu) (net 10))
 (segment (start 158.75 127) (end 166.37 127) (width 0.254) (layer B.Cu) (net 10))
 (segment (start 153.67 116.84) (end 161.29 109.22) (width 0.254) (layer B.Cu) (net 9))
 (segment (start 161.29 91.44) (end 161.29 91.44) (width 0.254) (layer B.Cu) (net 9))
 (segment (start 161.29 109.22) (end 161.29 91.44) (width 0.254) (layer B.Cu) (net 9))
 (segment (start 146.05 116.84) (end 153.67 116.84) (width 0.254) (layer B.Cu) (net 9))
 (segment (start 171.45 91.44) (end 171.704 91.44) (width 0.254) (layer F.Cu) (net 4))
 (segment (start 172.466 67.31) (end 165.1 67.31) (width 0.254) (layer F.Cu) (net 4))
 (segment (start 178.816 73.66) (end 172.466 67.31) (width 0.254) (layer F.Cu) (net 4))
 (segment (start 178.816 84.328) (end 178.816 73.66) (width 0.254) (layer F.Cu) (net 4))
 (segment (start 171.704 91.44) (end 178.816 84.328) (width 0.254) (layer F.Cu) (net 4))
 (segment (start 125.73 73.66) (end 116.84 73.66) (width 0.254) (layer B.Cu) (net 4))
 (segment (start 113.284 77.216) (end 113.284 83.439) (width 0.254) (layer B.Cu) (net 4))
 (segment (start 116.84 73.66) (end 113.284 77.216) (width 0.254) (layer B.Cu) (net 4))
 (segment (start 159.385 137.795) (end 153.67 132.08) (width 0.254) (layer B.Cu) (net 4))
 (segment (start 113.284 83.439) (end 117.475 87.63) (width 0.254) (layer B.Cu) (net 4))
 (segment (start 117.475 87.63) (end 117.475 123.825) (width 0.254) (layer B.Cu) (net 4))
 (segment (start 117.475 123.825) (end 137.16 143.51) (width 0.254) (layer B.Cu) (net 4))
 (segment (start 137.16 143.51) (end 161.29 143.51) (width 0.254) (layer B.Cu) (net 4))
 (segment (start 161.29 143.51) (end 159.385 141.605) (width 0.254) (layer B.Cu) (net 4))
 (segment (start 159.385 141.605) (end 159.385 137.795) (width 0.254) (layer B.Cu) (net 4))
 (segment (start 113.03 83.185) (end 113.284 83.439) (width 0.254) (layer B.Cu) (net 4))
 (segment (start 125.73 73.66) (end 125.73 76.2) (width 0.254) (layer B.Cu) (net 4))
 (segment (start 166.37 121.92) (end 172.085 121.92) (width 0.254) (layer F.Cu) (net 4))
 (segment (start 176.53 96.52) (end 171.45 91.44) (width 0.254) (layer F.Cu) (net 4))
 (segment (start 176.53 126.365) (end 176.53 96.52) (width 0.254) (layer F.Cu) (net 4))
 (segment (start 172.085 121.92) (end 176.53 126.365) (width 0.254) (layer F.Cu) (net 4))
 (segment (start 171.45 91.44) (end 169.545 91.44) (width 0.254) (layer F.Cu) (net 4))
 (segment (start 169.545 91.44) (end 168.91 92.075) (width 0.254) (layer F.Cu) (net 4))
 (segment (start 168.91 92.075) (end 168.91 91.44) (width 0.254) (layer F.Cu) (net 4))
 (segment (start 146.05 132.08) (end 146.05 131.445) (width 0.254) (layer F.Cu) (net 4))
 (segment (start 144.145 123.825) (end 146.05 121.92) (width 0.254) (layer F.Cu) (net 4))
 (segment (start 144.145 129.54) (end 144.145 123.825) (width 0.254) (layer F.Cu) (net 4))
 (segment (start 146.05 131.445) (end 144.145 129.54) (width 0.254) (layer F.Cu) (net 4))
 (segment (start 146.05 121.92) (end 142.875 121.92) (width 0.254) (layer F.Cu) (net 4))
 (segment (start 145.415 111.76) (end 146.05 111.76) (width 0.254) (layer F.Cu) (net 4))
 (segment (start 142.875 114.3) (end 142.875 121.92) (width 0.254) (layer F.Cu) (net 4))
 (segment (start 145.415 111.76) (end 142.875 114.3) (width 0.254) (layer F.Cu) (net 4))
 (segment (start 138.43 104.14) (end 146.05 111.76) (width 0.254) (layer F.Cu) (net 4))
 (segment (start 140.97 97.12) (end 140.97 101.6) (width 0.254) (layer F.Cu) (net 4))
 (segment (start 140.97 101.6) (end 138.43 104.14) (width 0.254) (layer F.Cu) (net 4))
 (segment (start 146.05 132.08) (end 153.67 132.08) (width 0.254) (layer B.Cu) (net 4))
 (segment (start 146.05 111.76) (end 153.67 111.76) (width 0.254) (layer B.Cu) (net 4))
 (segment (start 130.81 104.14) (end 138.43 104.14) (width 0.254) (layer B.Cu) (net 4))
 (segment (start 158.75 121.92) (end 166.37 121.92) (width 0.254) (layer B.Cu) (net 4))
 (segment (start 153.67 121.92) (end 158.75 121.92) (width 0.254) (layer B.Cu) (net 4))
 (segment (start 146.05 121.92) (end 153.67 121.92) (width 0.254) (layer B.Cu) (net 4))
 (segment (start 140.97 121.92) (end 146.05 121.92) (width 0.254) (layer B.Cu) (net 4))
 (segment (start 133.35 121.92) (end 140.97 121.92) (width 0.254) (layer B.Cu) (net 4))
 (segment (start 244.475 173.99) (end 244.475 176.149) (width 0.254) (layer F.Cu) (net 18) (status 400000))
 (segment (start 242.824 177.8) (end 241.554 177.8) (width 0.254) (layer F.Cu) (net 18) (status 800000))
 (segment (start 244.475 176.149) (end 242.824 177.8) (width 0.254) (layer F.Cu) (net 18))
 (segment (start 236.855 173.99) (end 236.855 176.911) (width 0.254) (layer F.Cu) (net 17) (status 400000))
 (segment (start 237.744 177.8) (end 239.014 177.8) (width 0.254) (layer F.Cu) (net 17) (status 800000))
 (segment (start 236.855 176.911) (end 237.744 177.8) (width 0.254) (layer F.Cu) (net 17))
 (segment (start 247.65 173.99) (end 247.65 179.07) (width 0.254) (layer F.Cu) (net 16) (status 400000))
 (segment (start 243.84 182.88) (end 241.554 182.88) (width 0.254) (layer F.Cu) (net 16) (status 800000))
 (segment (start 247.65 179.07) (end 243.84 182.88) (width 0.254) (layer F.Cu) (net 16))
 (segment (start 233.68 173.99) (end 233.68 178.816) (width 0.254) (layer F.Cu) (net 15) (status 400000))
 (segment (start 237.744 182.88) (end 239.014 182.88) (width 0.254) (layer F.Cu) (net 15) (status 800000))
 (segment (start 233.68 178.816) (end 237.744 182.88) (width 0.254) (layer F.Cu) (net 15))
 (segment (start 166.37 91.44) (end 166.37 84.582) (width 0.254) (layer F.Cu) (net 2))
 (segment (start 156.718 67.31) (end 162.56 67.31) (width 0.254) (layer F.Cu) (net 2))
 (segment (start 154.94 69.088) (end 156.718 67.31) (width 0.254) (layer F.Cu) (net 2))
 (segment (start 154.94 78.74) (end 154.94 69.088) (width 0.254) (layer F.Cu) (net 2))
 (segment (start 154.432 79.248) (end 154.94 78.74) (width 0.254) (layer F.Cu) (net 2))
 (segment (start 161.036 79.248) (end 154.432 79.248) (width 0.254) (layer F.Cu) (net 2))
 (segment (start 166.37 84.582) (end 161.036 79.248) (width 0.254) (layer F.Cu) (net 2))
 (segment (start 146.05 97.12) (end 146.05 96.266) (width 0.254) (layer F.Cu) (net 2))
 (segment (start 163.322 94.488) (end 166.37 91.44) (width 0.254) (layer F.Cu) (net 2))
 (segment (start 147.828 94.488) (end 163.322 94.488) (width 0.254) (layer F.Cu) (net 2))
 (segment (start 146.05 96.266) (end 147.828 94.488) (width 0.254) (layer F.Cu) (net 2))
 (segment (start 123.19 91.44) (end 123.19 93.726) (width 0.254) (layer B.Cu) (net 2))
 (segment (start 143.418 94.488) (end 146.05 97.12) (width 0.254) (layer F.Cu) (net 2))
 (segment (start 125.984 94.488) (end 143.418 94.488) (width 0.254) (layer F.Cu) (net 2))
 (segment (start 124.968 95.504) (end 125.984 94.488) (width 0.254) (layer F.Cu) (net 2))
 (via (at 124.968 95.504) (size 0.889) (layers F.Cu B.Cu) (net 2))
 (segment (start 123.19 93.726) (end 124.968 95.504) (width 0.254) (layer B.Cu) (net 2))
 (segment (start 123.19 76.2) (end 123.19 91.44) (width 0.254) (layer B.Cu) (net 2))
 (segment (start 162.56 67.31) (end 165.1 64.77) (width 0.254) (layer B.Cu) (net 2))
 (segment (start 128.27 73.66) (end 128.27 76.2) (width 0.254) (layer B.Cu) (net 19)))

